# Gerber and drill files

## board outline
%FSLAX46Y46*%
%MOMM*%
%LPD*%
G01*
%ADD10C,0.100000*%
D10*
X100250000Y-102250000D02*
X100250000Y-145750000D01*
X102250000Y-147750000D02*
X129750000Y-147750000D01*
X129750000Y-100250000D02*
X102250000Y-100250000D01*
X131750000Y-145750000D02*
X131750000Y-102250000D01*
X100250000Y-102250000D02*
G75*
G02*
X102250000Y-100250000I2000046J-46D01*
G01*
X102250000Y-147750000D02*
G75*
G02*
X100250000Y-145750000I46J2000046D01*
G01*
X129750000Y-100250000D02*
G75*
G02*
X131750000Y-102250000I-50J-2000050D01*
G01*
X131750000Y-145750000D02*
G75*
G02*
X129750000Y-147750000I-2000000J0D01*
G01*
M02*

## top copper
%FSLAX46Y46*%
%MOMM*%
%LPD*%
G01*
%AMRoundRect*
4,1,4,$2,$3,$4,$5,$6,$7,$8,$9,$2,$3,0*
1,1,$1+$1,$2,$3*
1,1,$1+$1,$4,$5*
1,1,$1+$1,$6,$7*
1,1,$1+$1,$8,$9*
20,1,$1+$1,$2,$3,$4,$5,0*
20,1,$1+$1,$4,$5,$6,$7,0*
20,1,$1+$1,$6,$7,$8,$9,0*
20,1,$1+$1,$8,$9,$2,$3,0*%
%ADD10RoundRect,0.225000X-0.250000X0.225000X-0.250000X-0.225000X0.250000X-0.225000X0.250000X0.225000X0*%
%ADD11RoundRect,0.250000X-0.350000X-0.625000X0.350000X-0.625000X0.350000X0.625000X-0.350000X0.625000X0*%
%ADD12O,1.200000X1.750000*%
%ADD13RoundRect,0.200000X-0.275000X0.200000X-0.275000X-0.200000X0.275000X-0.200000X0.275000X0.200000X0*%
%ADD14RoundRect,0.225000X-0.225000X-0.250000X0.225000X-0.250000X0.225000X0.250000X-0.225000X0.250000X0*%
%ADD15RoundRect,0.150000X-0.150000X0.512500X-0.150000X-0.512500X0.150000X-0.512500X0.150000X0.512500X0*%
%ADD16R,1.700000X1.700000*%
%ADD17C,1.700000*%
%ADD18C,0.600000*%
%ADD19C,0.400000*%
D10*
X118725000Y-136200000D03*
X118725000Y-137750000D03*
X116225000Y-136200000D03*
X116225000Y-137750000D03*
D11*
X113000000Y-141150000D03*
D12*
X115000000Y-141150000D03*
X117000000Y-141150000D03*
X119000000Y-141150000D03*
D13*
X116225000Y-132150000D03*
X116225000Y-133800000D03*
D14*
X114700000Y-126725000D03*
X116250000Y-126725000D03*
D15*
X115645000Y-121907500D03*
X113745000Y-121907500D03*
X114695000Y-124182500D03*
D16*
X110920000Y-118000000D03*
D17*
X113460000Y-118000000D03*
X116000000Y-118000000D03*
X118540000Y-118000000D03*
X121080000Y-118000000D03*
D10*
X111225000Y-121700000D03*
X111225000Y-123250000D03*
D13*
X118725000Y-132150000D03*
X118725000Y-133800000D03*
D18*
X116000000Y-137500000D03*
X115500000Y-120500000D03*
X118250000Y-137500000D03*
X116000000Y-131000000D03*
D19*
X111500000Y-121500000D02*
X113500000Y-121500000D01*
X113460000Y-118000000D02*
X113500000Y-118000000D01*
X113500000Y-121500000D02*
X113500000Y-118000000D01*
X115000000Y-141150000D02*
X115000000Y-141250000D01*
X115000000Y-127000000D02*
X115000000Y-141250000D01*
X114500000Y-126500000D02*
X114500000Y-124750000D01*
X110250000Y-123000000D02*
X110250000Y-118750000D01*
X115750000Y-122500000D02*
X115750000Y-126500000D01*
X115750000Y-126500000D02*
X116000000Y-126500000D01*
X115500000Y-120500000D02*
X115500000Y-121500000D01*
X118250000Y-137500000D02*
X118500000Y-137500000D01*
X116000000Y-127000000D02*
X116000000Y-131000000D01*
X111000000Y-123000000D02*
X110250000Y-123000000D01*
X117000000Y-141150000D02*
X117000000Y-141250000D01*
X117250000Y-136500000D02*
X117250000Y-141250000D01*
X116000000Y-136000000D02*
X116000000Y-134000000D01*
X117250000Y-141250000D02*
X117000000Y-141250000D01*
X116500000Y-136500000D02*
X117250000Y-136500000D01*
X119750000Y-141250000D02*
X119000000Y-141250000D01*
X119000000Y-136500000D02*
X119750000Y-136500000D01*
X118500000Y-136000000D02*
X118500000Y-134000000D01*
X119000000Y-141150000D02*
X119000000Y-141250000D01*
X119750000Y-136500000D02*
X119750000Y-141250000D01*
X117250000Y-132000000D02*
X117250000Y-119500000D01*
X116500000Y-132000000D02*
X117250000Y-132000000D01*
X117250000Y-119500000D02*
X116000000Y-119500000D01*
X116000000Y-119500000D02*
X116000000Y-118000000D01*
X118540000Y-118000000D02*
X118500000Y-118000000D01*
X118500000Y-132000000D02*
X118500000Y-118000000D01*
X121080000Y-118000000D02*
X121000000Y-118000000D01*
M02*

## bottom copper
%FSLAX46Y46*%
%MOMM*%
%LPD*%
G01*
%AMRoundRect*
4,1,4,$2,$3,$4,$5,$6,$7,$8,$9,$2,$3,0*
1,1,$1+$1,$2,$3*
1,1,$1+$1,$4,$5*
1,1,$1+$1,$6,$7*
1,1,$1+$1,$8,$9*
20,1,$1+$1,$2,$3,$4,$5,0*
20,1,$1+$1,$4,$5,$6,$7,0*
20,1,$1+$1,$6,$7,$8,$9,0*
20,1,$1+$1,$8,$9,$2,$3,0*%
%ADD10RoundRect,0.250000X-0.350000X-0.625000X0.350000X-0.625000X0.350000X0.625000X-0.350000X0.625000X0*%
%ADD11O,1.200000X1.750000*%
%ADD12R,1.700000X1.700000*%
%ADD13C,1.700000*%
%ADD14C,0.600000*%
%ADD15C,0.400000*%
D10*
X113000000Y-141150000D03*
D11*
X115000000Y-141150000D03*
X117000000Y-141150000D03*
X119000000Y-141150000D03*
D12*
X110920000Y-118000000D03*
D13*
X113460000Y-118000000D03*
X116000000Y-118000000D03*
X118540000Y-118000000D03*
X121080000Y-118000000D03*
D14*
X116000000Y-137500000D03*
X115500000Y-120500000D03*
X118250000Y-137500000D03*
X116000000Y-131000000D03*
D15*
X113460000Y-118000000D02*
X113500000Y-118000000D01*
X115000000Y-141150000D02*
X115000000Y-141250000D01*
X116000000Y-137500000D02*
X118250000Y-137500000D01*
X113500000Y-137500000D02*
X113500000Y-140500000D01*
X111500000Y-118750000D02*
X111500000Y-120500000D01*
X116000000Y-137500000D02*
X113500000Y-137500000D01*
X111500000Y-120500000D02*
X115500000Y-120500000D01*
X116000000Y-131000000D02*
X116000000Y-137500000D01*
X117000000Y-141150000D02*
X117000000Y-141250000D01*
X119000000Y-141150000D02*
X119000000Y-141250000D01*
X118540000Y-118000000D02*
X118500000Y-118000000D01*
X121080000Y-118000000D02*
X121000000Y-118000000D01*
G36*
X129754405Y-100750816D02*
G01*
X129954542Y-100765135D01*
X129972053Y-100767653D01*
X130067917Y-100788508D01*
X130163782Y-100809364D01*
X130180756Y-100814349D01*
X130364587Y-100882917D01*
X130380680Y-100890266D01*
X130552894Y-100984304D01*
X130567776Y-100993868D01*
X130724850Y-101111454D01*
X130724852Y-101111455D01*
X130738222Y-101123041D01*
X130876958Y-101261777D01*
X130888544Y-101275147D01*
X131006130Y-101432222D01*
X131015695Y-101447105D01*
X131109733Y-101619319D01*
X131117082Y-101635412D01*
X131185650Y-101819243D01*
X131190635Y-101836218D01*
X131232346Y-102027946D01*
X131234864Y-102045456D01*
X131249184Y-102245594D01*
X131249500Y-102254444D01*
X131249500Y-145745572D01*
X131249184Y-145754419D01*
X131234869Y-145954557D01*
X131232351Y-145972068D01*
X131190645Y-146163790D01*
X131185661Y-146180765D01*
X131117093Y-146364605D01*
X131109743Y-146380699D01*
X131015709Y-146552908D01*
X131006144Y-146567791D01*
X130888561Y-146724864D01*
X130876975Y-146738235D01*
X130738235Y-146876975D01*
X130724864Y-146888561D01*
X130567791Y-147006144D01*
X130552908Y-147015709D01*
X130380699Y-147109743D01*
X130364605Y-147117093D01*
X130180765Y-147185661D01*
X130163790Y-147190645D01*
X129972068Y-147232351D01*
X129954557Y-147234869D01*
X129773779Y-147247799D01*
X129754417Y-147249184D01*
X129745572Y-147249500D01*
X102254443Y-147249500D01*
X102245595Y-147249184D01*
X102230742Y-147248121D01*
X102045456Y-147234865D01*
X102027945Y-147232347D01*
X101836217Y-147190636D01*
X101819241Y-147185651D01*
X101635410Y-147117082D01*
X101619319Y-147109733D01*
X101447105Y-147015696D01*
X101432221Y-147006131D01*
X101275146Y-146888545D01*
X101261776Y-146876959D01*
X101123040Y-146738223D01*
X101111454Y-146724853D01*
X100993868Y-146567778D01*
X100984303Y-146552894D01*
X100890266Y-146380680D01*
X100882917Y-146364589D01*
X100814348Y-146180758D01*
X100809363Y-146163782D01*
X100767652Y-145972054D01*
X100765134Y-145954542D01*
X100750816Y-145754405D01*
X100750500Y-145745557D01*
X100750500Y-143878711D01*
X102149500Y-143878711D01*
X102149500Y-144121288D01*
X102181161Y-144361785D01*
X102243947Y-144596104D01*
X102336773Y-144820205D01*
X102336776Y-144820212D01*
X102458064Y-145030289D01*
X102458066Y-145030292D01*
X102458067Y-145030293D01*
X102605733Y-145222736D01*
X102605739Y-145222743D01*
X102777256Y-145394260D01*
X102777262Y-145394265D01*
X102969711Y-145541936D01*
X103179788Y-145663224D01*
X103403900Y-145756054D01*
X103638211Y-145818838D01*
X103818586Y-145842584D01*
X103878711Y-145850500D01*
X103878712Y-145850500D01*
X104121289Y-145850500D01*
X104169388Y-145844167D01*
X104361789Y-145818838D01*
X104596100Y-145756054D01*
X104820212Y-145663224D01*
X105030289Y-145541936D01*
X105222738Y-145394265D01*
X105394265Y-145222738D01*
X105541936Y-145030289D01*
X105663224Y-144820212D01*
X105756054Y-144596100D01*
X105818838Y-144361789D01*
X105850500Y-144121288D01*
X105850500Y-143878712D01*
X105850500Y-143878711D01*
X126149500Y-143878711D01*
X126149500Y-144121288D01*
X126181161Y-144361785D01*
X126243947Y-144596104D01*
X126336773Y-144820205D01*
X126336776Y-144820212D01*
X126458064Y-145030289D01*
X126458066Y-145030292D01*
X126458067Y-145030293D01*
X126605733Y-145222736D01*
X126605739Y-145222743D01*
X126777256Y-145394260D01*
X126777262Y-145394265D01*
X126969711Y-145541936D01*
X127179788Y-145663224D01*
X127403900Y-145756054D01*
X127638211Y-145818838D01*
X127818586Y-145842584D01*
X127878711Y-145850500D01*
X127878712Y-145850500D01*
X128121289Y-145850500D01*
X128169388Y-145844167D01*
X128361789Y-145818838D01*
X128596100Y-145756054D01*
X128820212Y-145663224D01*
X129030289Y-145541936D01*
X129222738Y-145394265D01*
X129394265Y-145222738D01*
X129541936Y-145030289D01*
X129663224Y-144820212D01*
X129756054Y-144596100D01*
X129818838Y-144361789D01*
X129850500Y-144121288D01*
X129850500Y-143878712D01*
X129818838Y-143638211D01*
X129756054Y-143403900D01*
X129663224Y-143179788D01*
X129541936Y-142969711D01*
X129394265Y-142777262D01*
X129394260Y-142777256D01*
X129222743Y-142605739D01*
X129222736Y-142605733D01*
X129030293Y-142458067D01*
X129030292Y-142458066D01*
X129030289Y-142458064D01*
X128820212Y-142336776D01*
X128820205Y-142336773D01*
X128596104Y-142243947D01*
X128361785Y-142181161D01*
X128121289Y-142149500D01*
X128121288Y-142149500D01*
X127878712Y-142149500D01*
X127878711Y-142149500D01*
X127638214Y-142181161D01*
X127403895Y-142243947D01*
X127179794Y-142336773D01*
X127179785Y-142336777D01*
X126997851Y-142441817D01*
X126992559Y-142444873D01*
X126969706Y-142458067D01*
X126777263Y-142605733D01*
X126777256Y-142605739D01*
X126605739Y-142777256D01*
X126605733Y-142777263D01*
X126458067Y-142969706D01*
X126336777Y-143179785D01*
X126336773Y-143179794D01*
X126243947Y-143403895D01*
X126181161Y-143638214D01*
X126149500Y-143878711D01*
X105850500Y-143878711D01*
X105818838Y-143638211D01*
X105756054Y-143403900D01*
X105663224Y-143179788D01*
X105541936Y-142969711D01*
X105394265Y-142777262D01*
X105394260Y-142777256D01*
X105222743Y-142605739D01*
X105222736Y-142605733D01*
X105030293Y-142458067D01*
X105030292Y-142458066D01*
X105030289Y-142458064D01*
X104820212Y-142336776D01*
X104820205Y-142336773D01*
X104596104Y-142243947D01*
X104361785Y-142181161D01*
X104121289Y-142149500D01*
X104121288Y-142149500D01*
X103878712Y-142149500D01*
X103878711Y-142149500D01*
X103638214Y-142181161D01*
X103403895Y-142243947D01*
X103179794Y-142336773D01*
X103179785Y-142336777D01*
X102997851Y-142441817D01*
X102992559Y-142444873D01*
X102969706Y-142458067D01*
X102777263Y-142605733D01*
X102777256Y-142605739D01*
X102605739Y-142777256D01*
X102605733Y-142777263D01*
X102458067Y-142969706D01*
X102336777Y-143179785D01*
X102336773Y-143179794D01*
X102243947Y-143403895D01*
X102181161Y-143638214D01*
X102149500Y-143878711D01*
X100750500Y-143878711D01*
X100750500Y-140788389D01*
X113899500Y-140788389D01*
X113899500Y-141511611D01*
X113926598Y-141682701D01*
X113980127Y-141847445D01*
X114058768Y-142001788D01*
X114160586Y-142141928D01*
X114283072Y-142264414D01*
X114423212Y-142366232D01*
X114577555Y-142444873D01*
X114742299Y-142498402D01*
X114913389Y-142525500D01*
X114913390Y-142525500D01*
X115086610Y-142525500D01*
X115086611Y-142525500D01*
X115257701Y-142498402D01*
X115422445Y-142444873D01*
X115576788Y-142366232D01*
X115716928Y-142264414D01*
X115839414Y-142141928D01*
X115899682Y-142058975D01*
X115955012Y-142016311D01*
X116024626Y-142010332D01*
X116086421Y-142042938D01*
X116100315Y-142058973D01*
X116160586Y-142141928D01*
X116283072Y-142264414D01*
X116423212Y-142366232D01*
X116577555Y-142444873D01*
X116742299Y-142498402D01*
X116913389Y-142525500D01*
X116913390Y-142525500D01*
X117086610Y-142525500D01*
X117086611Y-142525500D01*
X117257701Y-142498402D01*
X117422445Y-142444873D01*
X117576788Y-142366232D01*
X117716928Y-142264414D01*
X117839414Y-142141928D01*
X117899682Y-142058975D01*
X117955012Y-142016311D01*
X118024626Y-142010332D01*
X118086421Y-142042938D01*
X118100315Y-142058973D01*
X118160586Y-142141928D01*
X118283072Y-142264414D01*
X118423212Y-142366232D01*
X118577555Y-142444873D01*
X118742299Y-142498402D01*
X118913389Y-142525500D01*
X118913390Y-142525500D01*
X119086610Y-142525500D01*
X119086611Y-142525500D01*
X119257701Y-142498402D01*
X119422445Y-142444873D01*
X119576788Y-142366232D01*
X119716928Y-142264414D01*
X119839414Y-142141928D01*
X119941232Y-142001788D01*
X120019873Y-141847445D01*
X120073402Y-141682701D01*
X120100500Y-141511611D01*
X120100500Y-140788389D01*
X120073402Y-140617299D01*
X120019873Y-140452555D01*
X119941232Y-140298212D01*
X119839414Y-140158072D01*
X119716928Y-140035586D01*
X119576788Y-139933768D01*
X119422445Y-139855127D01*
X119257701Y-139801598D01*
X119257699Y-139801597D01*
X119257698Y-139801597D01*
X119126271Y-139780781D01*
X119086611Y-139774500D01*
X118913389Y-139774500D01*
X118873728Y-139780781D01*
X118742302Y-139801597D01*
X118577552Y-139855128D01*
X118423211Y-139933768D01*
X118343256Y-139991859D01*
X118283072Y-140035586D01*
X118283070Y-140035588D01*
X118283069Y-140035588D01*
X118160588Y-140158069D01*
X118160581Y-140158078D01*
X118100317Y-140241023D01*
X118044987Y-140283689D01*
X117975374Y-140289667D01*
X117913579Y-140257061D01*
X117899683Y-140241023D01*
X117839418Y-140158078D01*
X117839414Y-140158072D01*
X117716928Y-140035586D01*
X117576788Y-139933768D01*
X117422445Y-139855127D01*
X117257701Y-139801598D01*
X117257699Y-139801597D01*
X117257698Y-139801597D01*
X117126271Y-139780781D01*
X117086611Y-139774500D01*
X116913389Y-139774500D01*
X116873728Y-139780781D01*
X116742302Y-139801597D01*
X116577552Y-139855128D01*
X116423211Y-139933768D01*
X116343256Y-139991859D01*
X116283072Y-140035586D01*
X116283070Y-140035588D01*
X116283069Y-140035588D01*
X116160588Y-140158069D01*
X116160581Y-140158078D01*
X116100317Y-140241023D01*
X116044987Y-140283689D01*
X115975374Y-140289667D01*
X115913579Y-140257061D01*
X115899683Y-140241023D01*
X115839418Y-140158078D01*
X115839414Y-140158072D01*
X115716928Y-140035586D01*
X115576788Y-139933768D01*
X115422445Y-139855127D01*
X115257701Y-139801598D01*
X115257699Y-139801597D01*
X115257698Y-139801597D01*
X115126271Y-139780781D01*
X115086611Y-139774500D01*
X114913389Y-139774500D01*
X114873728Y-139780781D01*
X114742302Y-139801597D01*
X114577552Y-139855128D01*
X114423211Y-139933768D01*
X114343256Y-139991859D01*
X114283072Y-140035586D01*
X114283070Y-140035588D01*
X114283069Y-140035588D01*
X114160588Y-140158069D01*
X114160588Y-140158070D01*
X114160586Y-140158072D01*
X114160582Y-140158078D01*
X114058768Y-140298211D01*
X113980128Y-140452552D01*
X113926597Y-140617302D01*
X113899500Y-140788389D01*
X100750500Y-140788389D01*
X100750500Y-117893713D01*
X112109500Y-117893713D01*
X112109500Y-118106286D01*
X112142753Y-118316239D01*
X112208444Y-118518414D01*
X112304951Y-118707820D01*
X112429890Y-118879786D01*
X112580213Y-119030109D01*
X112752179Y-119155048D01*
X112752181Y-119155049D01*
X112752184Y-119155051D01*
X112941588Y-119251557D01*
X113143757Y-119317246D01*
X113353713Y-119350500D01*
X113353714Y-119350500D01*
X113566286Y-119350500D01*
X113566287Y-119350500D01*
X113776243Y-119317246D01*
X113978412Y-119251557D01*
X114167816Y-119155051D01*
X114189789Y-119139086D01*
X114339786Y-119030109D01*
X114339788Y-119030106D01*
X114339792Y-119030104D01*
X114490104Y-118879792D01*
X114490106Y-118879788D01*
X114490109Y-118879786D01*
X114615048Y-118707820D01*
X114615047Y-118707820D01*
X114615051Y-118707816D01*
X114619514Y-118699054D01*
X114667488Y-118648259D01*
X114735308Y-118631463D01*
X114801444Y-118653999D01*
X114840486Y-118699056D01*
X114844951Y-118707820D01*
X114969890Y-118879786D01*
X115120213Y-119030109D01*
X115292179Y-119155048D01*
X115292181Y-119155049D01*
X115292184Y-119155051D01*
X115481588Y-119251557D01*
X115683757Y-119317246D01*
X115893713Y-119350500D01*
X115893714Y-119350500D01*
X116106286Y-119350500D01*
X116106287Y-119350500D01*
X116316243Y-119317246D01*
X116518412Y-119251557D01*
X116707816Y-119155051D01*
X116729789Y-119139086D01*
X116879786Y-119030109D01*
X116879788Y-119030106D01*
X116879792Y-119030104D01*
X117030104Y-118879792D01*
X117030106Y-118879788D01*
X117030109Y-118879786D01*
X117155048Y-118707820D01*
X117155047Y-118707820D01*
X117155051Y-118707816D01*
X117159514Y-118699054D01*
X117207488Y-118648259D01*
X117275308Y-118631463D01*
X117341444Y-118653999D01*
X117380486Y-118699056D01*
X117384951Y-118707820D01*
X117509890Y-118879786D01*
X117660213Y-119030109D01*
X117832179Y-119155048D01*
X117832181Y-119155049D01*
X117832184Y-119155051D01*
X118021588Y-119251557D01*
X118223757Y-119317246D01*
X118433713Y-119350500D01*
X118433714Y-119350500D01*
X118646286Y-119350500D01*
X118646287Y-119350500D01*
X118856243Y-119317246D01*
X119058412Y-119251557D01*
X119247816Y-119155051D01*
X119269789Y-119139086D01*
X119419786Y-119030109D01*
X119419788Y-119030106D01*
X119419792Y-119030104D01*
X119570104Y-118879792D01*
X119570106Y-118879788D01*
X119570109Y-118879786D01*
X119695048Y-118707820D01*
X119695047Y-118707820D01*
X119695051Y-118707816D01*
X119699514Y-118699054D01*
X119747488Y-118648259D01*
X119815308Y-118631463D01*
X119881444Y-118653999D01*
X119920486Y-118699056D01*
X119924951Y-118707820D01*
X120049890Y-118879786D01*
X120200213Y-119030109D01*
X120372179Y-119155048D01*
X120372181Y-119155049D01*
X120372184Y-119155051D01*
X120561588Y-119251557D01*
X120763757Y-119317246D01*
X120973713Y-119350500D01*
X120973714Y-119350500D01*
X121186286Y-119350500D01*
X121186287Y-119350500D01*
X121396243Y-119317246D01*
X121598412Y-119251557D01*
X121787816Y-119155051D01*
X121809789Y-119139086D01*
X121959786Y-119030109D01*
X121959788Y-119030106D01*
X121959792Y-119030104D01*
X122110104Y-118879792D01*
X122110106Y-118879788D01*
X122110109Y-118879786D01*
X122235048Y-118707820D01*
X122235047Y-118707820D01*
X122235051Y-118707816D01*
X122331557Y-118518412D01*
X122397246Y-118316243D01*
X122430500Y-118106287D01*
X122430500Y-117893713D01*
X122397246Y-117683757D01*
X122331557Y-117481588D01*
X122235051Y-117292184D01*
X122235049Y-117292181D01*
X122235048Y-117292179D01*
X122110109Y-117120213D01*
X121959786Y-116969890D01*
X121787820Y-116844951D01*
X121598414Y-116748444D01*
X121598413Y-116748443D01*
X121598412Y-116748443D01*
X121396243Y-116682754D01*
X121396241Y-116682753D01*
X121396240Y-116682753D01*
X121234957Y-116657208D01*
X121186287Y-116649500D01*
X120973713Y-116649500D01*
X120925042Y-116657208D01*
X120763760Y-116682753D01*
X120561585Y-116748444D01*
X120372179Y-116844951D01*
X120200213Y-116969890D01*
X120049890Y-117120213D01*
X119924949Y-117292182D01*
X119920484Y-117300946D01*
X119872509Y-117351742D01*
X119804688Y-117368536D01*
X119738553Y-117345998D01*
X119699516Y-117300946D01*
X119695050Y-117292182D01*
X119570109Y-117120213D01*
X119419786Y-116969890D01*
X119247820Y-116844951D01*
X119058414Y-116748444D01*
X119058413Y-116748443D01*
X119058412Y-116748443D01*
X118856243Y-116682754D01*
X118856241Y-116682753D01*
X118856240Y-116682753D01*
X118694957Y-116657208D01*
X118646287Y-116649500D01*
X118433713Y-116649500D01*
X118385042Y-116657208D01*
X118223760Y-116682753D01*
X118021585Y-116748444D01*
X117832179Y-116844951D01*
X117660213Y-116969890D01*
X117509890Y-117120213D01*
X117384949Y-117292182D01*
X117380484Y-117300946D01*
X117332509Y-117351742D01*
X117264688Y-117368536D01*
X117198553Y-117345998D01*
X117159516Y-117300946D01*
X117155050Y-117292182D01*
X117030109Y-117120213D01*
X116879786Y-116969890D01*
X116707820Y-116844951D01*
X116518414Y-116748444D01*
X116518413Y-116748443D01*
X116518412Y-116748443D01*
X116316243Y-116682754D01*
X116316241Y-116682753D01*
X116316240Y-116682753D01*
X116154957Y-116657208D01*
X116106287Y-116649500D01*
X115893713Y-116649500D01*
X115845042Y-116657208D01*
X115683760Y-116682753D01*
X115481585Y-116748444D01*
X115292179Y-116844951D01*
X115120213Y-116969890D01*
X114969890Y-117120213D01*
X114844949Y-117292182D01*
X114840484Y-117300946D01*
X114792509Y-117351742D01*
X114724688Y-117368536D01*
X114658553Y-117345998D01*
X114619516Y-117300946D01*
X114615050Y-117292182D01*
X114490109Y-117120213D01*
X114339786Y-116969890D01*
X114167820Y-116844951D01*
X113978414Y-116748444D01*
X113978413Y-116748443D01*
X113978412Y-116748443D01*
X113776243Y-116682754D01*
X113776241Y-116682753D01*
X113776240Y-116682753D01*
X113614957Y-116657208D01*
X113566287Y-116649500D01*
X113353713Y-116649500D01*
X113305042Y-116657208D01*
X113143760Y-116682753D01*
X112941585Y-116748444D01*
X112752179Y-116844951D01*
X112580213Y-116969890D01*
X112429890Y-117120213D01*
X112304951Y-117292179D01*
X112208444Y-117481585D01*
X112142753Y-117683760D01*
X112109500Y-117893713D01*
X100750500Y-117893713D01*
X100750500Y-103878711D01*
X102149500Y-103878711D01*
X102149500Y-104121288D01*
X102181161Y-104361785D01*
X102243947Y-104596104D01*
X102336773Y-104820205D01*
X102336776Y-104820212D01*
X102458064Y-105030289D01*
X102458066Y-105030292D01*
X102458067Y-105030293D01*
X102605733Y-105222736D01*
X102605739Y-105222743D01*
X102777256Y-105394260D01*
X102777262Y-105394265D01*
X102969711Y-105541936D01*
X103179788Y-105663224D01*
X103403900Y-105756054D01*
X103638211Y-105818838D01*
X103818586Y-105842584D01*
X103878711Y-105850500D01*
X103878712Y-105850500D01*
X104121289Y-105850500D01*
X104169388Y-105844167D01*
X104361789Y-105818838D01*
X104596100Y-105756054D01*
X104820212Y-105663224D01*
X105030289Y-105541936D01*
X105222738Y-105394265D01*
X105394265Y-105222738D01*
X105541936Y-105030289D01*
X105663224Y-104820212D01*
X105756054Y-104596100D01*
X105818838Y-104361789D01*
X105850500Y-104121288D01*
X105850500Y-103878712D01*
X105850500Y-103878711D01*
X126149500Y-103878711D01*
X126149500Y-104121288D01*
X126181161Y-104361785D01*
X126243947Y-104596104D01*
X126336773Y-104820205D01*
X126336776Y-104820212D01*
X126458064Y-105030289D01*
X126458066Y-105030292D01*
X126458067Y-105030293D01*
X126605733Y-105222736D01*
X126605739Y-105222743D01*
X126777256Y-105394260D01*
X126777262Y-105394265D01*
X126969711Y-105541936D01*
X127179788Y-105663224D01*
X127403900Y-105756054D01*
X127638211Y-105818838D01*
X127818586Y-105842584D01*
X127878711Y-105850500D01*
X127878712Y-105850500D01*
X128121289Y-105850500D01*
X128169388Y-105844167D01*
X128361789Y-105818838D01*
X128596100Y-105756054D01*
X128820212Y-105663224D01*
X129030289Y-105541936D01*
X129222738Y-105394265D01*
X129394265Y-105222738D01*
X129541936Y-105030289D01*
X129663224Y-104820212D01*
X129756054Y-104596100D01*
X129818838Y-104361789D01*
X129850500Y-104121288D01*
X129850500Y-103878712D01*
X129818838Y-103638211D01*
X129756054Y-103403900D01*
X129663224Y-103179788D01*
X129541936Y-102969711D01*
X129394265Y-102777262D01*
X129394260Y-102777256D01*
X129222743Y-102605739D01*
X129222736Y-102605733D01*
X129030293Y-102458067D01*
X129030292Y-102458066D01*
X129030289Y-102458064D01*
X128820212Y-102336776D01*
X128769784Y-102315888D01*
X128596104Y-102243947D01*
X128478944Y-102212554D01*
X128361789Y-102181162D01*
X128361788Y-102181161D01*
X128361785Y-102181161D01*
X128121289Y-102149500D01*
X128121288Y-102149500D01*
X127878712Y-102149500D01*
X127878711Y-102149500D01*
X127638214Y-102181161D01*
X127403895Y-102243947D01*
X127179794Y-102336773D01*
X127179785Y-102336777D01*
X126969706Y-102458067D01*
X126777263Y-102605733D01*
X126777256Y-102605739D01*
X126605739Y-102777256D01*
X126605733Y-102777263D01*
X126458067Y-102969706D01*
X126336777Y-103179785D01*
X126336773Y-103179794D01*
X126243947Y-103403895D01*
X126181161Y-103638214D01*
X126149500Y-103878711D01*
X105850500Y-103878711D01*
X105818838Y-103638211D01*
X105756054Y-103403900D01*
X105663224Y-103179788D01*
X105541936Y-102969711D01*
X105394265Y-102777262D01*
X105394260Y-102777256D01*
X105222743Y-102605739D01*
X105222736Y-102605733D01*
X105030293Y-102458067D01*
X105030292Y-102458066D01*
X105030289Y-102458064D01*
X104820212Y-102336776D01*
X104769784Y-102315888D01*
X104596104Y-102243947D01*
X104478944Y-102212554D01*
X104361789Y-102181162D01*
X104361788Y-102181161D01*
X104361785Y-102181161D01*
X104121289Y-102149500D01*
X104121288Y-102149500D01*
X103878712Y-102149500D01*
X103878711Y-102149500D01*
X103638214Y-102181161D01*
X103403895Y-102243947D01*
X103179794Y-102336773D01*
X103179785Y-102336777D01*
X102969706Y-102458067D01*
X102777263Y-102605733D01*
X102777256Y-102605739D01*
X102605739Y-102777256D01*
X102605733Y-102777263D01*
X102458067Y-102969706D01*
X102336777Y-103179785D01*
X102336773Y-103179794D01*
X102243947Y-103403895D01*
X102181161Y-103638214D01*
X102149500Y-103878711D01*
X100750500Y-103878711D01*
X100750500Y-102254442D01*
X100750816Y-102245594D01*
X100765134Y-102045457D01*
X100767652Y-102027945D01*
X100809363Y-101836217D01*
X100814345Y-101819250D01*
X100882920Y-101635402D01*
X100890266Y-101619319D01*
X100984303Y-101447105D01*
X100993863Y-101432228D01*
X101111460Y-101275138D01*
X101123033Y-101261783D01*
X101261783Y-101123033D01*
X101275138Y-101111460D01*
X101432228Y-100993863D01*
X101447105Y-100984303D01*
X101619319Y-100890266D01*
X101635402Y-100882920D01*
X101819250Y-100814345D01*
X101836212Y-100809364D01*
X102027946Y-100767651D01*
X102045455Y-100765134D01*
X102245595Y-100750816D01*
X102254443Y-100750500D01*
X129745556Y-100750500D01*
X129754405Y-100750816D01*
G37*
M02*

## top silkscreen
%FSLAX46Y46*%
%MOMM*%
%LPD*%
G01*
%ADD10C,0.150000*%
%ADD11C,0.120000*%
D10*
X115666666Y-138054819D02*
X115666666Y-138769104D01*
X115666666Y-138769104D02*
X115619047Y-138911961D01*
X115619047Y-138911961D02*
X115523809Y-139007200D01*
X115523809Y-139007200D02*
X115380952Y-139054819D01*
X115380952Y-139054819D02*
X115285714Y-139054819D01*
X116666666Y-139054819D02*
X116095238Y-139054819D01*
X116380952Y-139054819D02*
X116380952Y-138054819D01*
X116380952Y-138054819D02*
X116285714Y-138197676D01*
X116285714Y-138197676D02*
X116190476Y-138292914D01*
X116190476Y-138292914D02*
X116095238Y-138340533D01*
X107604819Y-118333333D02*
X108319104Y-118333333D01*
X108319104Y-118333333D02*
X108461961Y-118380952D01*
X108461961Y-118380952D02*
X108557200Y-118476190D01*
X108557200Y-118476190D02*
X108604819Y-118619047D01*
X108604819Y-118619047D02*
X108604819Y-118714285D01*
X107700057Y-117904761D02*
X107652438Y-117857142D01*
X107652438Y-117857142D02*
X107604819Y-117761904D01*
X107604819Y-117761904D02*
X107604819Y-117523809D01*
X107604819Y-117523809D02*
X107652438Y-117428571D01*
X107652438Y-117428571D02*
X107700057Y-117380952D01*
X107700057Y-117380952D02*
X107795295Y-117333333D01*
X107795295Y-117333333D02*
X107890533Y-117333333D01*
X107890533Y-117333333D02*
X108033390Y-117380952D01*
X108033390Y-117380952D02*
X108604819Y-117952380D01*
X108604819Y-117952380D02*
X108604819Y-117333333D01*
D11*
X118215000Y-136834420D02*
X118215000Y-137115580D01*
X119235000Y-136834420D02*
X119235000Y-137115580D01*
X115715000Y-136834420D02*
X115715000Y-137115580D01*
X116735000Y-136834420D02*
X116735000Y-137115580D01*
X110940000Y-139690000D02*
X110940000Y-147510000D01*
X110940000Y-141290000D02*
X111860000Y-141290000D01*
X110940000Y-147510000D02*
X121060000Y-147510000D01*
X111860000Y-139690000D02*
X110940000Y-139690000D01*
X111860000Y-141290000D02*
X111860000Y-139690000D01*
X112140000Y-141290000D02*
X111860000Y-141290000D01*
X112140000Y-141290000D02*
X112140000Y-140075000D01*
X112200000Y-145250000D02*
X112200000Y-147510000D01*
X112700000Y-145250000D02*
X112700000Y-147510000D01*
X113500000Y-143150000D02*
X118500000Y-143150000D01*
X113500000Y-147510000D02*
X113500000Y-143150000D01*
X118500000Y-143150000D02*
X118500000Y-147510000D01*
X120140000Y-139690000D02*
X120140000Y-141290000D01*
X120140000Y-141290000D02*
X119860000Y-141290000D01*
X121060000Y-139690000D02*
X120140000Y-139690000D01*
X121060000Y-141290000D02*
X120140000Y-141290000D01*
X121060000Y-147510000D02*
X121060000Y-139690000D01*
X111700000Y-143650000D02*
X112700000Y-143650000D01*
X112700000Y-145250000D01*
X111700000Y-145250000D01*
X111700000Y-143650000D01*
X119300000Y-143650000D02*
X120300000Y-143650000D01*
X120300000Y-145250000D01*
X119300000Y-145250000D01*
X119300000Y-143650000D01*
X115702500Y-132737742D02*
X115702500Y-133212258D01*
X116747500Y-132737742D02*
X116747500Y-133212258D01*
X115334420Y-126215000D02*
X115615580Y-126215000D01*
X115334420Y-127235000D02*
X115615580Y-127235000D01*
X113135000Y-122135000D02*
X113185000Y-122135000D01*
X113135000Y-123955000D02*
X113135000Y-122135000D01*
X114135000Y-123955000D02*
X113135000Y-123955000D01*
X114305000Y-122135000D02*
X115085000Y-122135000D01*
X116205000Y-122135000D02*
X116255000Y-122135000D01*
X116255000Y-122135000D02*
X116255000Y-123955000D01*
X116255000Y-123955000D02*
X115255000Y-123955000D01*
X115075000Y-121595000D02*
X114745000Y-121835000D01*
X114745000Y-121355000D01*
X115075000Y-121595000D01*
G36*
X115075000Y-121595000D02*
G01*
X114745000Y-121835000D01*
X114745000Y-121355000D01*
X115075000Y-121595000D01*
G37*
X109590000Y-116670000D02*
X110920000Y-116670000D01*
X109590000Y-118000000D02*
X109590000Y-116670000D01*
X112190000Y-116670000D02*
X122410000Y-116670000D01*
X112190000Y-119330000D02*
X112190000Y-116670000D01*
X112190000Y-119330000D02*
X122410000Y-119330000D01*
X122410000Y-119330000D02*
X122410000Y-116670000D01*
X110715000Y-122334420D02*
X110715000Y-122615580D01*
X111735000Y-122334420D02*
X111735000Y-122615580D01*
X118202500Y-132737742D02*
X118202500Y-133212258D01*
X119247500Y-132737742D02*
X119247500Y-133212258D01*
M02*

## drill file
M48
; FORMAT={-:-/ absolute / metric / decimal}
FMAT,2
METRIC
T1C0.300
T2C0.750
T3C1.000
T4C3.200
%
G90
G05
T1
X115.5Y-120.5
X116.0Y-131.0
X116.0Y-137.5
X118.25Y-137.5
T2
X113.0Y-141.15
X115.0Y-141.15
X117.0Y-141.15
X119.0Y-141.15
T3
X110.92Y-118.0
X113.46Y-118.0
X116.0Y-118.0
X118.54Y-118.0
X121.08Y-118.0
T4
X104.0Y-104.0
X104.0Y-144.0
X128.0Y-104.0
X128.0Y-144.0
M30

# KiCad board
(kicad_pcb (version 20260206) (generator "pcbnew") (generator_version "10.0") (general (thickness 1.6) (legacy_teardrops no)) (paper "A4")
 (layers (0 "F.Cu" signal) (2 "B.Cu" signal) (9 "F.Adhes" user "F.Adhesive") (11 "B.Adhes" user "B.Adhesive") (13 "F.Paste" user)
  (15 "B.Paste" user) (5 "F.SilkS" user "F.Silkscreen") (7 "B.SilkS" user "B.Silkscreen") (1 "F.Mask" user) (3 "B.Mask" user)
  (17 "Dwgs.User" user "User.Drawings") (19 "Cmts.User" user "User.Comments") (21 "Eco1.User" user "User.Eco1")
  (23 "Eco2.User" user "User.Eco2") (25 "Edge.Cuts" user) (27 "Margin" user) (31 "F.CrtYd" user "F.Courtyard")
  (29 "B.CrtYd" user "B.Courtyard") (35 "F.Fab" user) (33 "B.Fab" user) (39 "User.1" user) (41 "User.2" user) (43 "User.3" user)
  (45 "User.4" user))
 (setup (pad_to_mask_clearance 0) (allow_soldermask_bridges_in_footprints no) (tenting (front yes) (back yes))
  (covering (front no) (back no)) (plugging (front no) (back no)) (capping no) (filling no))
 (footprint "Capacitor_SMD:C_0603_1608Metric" (layer "F.Cu") (at 118.725 136.975 -90)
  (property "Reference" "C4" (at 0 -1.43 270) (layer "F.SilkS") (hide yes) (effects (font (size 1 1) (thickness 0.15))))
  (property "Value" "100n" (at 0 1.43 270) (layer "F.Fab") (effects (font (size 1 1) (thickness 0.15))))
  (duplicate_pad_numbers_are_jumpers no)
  (fp_line (start -0.14058 0.51) (end 0.14058 0.51) (stroke (width 0.12) (type solid)) (layer "F.SilkS"))
  (fp_line (start -0.14058 -0.51) (end 0.14058 -0.51) (stroke (width 0.12) (type solid)) (layer "F.SilkS"))
  (pad "1" smd roundrect (at -0.775 0 270) (size 0.9 0.95) (layers "F.Cu" "F.Mask" "F.Paste") (roundrect_rratio 0.25) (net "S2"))
  (pad "2" smd roundrect (at 0.775 0 270) (size 0.9 0.95) (layers "F.Cu" "F.Mask" "F.Paste") (roundrect_rratio 0.25) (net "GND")))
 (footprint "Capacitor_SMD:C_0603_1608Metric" (layer "F.Cu") (at 116.225 136.975 -90)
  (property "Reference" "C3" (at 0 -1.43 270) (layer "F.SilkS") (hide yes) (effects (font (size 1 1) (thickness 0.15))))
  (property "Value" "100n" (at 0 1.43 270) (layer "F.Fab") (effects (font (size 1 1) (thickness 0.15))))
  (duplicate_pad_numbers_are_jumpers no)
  (fp_line (start -0.14058 0.51) (end 0.14058 0.51) (stroke (width 0.12) (type solid)) (layer "F.SilkS"))
  (fp_line (start -0.14058 -0.51) (end 0.14058 -0.51) (stroke (width 0.12) (type solid)) (layer "F.SilkS"))
  (pad "1" smd roundrect (at -0.775 0 270) (size 0.9 0.95) (layers "F.Cu" "F.Mask" "F.Paste") (roundrect_rratio 0.25) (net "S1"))
  (pad "2" smd roundrect (at 0.775 0 270) (size 0.9 0.95) (layers "F.Cu" "F.Mask" "F.Paste") (roundrect_rratio 0.25) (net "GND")))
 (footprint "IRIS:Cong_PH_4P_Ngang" (layer "F.Cu") (at 113 141.15)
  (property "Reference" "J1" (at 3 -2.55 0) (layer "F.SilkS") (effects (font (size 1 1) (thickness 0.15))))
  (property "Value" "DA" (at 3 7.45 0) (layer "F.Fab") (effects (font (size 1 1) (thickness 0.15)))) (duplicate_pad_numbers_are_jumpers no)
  (fp_line (start -2.06 -1.46) (end -2.06 6.36) (stroke (width 0.12) (type solid)) (layer "F.SilkS"))
  (fp_line (start -2.06 0.14) (end -1.14 0.14) (stroke (width 0.12) (type solid)) (layer "F.SilkS"))
  (fp_line (start -2.06 6.36) (end 8.06 6.36) (stroke (width 0.12) (type solid)) (layer "F.SilkS"))
  (fp_line (start -1.14 -1.46) (end -2.06 -1.46) (stroke (width 0.12) (type solid)) (layer "F.SilkS"))
  (fp_line (start -1.14 0.14) (end -1.14 -1.46) (stroke (width 0.12) (type solid)) (layer "F.SilkS"))
  (fp_line (start -0.86 0.14) (end -1.14 0.14) (stroke (width 0.12) (type solid)) (layer "F.SilkS"))
  (fp_line (start -0.86 0.14) (end -0.86 -1.075) (stroke (width 0.12) (type solid)) (layer "F.SilkS"))
  (fp_line (start -0.8 4.1) (end -0.8 6.36) (stroke (width 0.12) (type solid)) (layer "F.SilkS"))
  (fp_line (start -0.3 4.1) (end -0.3 6.36) (stroke (width 0.12) (type solid)) (layer "F.SilkS"))
  (fp_line (start 0.5 2) (end 5.5 2) (stroke (width 0.12) (type solid)) (layer "F.SilkS"))
  (fp_line (start 0.5 6.36) (end 0.5 2) (stroke (width 0.12) (type solid)) (layer "F.SilkS"))
  (fp_line (start 5.5 2) (end 5.5 6.36) (stroke (width 0.12) (type solid)) (layer "F.SilkS"))
  (fp_line (start 7.14 -1.46) (end 7.14 0.14) (stroke (width 0.12) (type solid)) (layer "F.SilkS"))
  (fp_line (start 7.14 0.14) (end 6.86 0.14) (stroke (width 0.12) (type solid)) (layer "F.SilkS"))
  (fp_line (start 8.06 -1.46) (end 7.14 -1.46) (stroke (width 0.12) (type solid)) (layer "F.SilkS"))
  (fp_line (start 8.06 0.14) (end 7.14 0.14) (stroke (width 0.12) (type solid)) (layer "F.SilkS"))
  (fp_line (start 8.06 6.36) (end 8.06 -1.46) (stroke (width 0.12) (type solid)) (layer "F.SilkS"))
  (fp_rect (start -1.3 2.5) (end -0.3 4.1) (stroke (width 0.12) (type solid)) (fill no) (layer "F.SilkS"))
  (fp_rect (start 6.3 2.5) (end 7.3 4.1) (stroke (width 0.12) (type solid)) (fill no) (layer "F.SilkS"))
  (pad "1" thru_hole roundrect (at 0 0) (size 1.2 1.75) (drill 0.75) (layers "*.Cu" "*.Mask") (remove_unused_layers no)
   (roundrect_rratio 0.208333) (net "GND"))
  (pad "2" thru_hole oval (at 2 0) (size 1.2 1.75) (drill 0.75) (layers "*.Cu" "*.Mask") (remove_unused_layers no) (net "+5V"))
  (pad "3" thru_hole oval (at 4 0) (size 1.2 1.75) (drill 0.75) (layers "*.Cu" "*.Mask") (remove_unused_layers no) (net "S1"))
  (pad "4" thru_hole oval (at 6 0) (size 1.2 1.75) (drill 0.75) (layers "*.Cu" "*.Mask") (remove_unused_layers no) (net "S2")))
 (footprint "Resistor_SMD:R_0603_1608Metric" (layer "F.Cu") (at 116.225 132.975 -90)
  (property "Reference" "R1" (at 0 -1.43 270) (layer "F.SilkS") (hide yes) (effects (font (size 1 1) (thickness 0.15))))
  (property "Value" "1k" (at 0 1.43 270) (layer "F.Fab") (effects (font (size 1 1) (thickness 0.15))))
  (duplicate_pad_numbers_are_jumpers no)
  (fp_line (start -0.237258 0.5225) (end 0.237258 0.5225) (stroke (width 0.12) (type solid)) (layer "F.SilkS"))
  (fp_line (start -0.237258 -0.5225) (end 0.237258 -0.5225) (stroke (width 0.12) (type solid)) (layer "F.SilkS"))
  (pad "1" smd roundrect (at -0.825 0 270) (size 0.8 0.95) (layers "F.Cu" "F.Mask" "F.Paste") (roundrect_rratio 0.25) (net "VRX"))
  (pad "2" smd roundrect (at 0.825 0 270) (size 0.8 0.95) (layers "F.Cu" "F.Mask" "F.Paste") (roundrect_rratio 0.25) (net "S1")))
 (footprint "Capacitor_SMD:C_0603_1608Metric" (layer "F.Cu") (at 115.475 126.725)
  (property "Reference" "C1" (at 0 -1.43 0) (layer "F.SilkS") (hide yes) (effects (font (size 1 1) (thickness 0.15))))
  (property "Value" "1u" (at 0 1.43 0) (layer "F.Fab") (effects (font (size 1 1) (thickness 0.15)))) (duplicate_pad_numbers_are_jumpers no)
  (fp_line (start -0.14058 -0.51) (end 0.14058 -0.51) (stroke (width 0.12) (type solid)) (layer "F.SilkS"))
  (fp_line (start -0.14058 0.51) (end 0.14058 0.51) (stroke (width 0.12) (type solid)) (layer "F.SilkS"))
  (pad "1" smd roundrect (at -0.775 0) (size 0.9 0.95) (layers "F.Cu" "F.Mask" "F.Paste") (roundrect_rratio 0.25) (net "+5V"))
  (pad "2" smd roundrect (at 0.775 0) (size 0.9 0.95) (layers "F.Cu" "F.Mask" "F.Paste") (roundrect_rratio 0.25) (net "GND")))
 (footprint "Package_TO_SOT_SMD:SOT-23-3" (layer "F.Cu") (at 114.695 123.045 -90)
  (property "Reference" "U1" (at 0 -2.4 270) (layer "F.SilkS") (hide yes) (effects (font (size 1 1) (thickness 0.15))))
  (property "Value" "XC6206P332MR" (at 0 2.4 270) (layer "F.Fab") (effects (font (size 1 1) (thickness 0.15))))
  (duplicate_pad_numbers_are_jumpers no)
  (fp_line (start -0.91 1.56) (end -0.91 1.51) (stroke (width 0.12) (type solid)) (layer "F.SilkS"))
  (fp_line (start 0.91 1.56) (end -0.91 1.56) (stroke (width 0.12) (type solid)) (layer "F.SilkS"))
  (fp_line (start 0.91 0.56) (end 0.91 1.56) (stroke (width 0.12) (type solid)) (layer "F.SilkS"))
  (fp_line (start -0.91 0.39) (end -0.91 -0.39) (stroke (width 0.12) (type solid)) (layer "F.SilkS"))
  (fp_line (start -0.91 -1.51) (end -0.91 -1.56) (stroke (width 0.12) (type solid)) (layer "F.SilkS"))
  (fp_line (start -0.91 -1.56) (end 0.91 -1.56) (stroke (width 0.12) (type solid)) (layer "F.SilkS"))
  (fp_line (start 0.91 -1.56) (end 0.91 -0.56) (stroke (width 0.12) (type solid)) (layer "F.SilkS"))
  (fp_poly (pts (xy -1.45 -0.38) (xy -1.21 -0.05) (xy -1.69 -0.05)) (stroke (width 0.12) (type solid)) (fill yes) (layer "F.SilkS"))
  (pad "1" smd roundrect (at -1.1375 -0.95 270) (size 1.325 0.6) (layers "F.Cu" "F.Mask" "F.Paste") (roundrect_rratio 0.25) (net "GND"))
  (pad "2" smd roundrect (at -1.1375 0.95 270) (size 1.325 0.6) (layers "F.Cu" "F.Mask" "F.Paste") (roundrect_rratio 0.25) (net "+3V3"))
  (pad "3" smd roundrect (at 1.1375 0 270) (size 1.325 0.6) (layers "F.Cu" "F.Mask" "F.Paste") (roundrect_rratio 0.25) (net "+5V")))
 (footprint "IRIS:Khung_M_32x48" (layer "F.Cu") (at 100 148)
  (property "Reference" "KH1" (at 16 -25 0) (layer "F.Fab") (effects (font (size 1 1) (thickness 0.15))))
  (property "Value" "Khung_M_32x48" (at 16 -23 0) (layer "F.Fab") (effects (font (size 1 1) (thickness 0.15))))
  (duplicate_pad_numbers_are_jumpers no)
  (fp_line (start 0.25 -45.75) (end 0.25 -2.25) (stroke (width 0.1) (type solid)) (layer "Edge.Cuts"))
  (fp_line (start 2.25 -0.25) (end 29.75 -0.25) (stroke (width 0.1) (type solid)) (layer "Edge.Cuts"))
  (fp_line (start 29.75 -47.75) (end 2.25 -47.75) (stroke (width 0.1) (type solid)) (layer "Edge.Cuts"))
  (fp_line (start 31.75 -2.25) (end 31.75 -45.75) (stroke (width 0.1) (type solid)) (layer "Edge.Cuts"))
  (fp_arc (start 0.25 -45.75) (mid 0.8358 -47.1642) (end 2.25 -47.75) (stroke (width 0.1) (type solid)) (layer "Edge.Cuts"))
  (fp_arc (start 2.25 -0.25) (mid 0.8358 -0.8358) (end 0.25 -2.25) (stroke (width 0.1) (type solid)) (layer "Edge.Cuts"))
  (fp_arc (start 29.75 -47.75) (mid 31.164199 -47.164199) (end 31.75 -45.75) (stroke (width 0.1) (type solid)) (layer "Edge.Cuts"))
  (fp_arc (start 31.75 -2.25) (mid 31.164214 -0.835786) (end 29.75 -0.25) (stroke (width 0.1) (type solid)) (layer "Edge.Cuts"))
  (pad "" np_thru_hole circle (at 4 -44) (size 3.2 3.2) (drill 3.2) (layers "*.Cu" "*.Mask"))
  (pad "" np_thru_hole circle (at 4 -4) (size 3.2 3.2) (drill 3.2) (layers "*.Cu" "*.Mask"))
  (pad "" np_thru_hole circle (at 28 -44) (size 3.2 3.2) (drill 3.2) (layers "*.Cu" "*.Mask"))
  (pad "" np_thru_hole circle (at 28 -4) (size 3.2 3.2) (drill 3.2) (layers "*.Cu" "*.Mask")))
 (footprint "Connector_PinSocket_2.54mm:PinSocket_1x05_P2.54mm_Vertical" (layer "F.Cu") (at 110.92 118 90)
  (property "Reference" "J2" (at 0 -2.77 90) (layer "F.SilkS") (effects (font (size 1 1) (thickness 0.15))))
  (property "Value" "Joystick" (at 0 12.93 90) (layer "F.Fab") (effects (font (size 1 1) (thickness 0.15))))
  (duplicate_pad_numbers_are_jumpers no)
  (fp_line (start 1.33 -1.33) (end 1.33 0) (stroke (width 0.12) (type solid)) (layer "F.SilkS"))
  (fp_line (start 0 -1.33) (end 1.33 -1.33) (stroke (width 0.12) (type solid)) (layer "F.SilkS"))
  (fp_line (start 1.33 1.27) (end 1.33 11.49) (stroke (width 0.12) (type solid)) (layer "F.SilkS"))
  (fp_line (start -1.33 1.27) (end 1.33 1.27) (stroke (width 0.12) (type solid)) (layer "F.SilkS"))
  (fp_line (start -1.33 1.27) (end -1.33 11.49) (stroke (width 0.12) (type solid)) (layer "F.SilkS"))
  (fp_line (start -1.33 11.49) (end 1.33 11.49) (stroke (width 0.12) (type solid)) (layer "F.SilkS"))
  (pad "1" thru_hole rect (at 0 0 90) (size 1.7 1.7) (drill 1) (layers "*.Cu" "*.Mask") (remove_unused_layers no) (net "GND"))
  (pad "2" thru_hole circle (at 0 2.54 90) (size 1.7 1.7) (drill 1) (layers "*.Cu" "*.Mask") (remove_unused_layers no) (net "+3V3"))
  (pad "3" thru_hole circle (at 0 5.08 90) (size 1.7 1.7) (drill 1) (layers "*.Cu" "*.Mask") (remove_unused_layers no) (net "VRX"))
  (pad "4" thru_hole circle (at 0 7.62 90) (size 1.7 1.7) (drill 1) (layers "*.Cu" "*.Mask") (remove_unused_layers no) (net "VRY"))
  (pad "5" thru_hole circle (at 0 10.16 90) (size 1.7 1.7) (drill 1) (layers "*.Cu" "*.Mask") (remove_unused_layers no)
   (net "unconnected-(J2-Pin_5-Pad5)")))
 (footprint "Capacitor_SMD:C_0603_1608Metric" (layer "F.Cu") (at 111.225 122.475 -90)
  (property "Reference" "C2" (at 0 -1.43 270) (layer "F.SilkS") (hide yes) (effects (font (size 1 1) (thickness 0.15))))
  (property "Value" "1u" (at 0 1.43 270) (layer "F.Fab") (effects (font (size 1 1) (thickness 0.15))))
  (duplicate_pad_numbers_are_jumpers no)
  (fp_line (start -0.14058 0.51) (end 0.14058 0.51) (stroke (width 0.12) (type solid)) (layer "F.SilkS"))
  (fp_line (start -0.14058 -0.51) (end 0.14058 -0.51) (stroke (width 0.12) (type solid)) (layer "F.SilkS"))
  (pad "1" smd roundrect (at -0.775 0 270) (size 0.9 0.95) (layers "F.Cu" "F.Mask" "F.Paste") (roundrect_rratio 0.25) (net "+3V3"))
  (pad "2" smd roundrect (at 0.775 0 270) (size 0.9 0.95) (layers "F.Cu" "F.Mask" "F.Paste") (roundrect_rratio 0.25) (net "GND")))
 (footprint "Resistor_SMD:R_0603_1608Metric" (layer "F.Cu") (at 118.725 132.975 -90)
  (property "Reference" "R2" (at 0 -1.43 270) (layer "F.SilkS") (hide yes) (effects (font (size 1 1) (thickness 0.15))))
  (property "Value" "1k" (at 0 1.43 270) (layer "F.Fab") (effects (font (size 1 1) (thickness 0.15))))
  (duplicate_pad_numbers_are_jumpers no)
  (fp_line (start -0.237258 0.5225) (end 0.237258 0.5225) (stroke (width 0.12) (type solid)) (layer "F.SilkS"))
  (fp_line (start -0.237258 -0.5225) (end 0.237258 -0.5225) (stroke (width 0.12) (type solid)) (layer "F.SilkS"))
  (pad "1" smd roundrect (at -0.825 0 270) (size 0.8 0.95) (layers "F.Cu" "F.Mask" "F.Paste") (roundrect_rratio 0.25) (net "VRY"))
  (pad "2" smd roundrect (at 0.825 0 270) (size 0.8 0.95) (layers "F.Cu" "F.Mask" "F.Paste") (roundrect_rratio 0.25) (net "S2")))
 (segment (start 111.5 121.5) (end 113.5 121.5) (width 0.4) (layer "F.Cu") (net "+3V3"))
 (segment (start 113.46 118) (end 113.5 118) (width 0.4) (layer "F.Cu") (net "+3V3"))
 (segment (start 113.5 121.5) (end 113.5 118) (width 0.4) (layer "F.Cu") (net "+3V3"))
 (segment (start 113.46 118) (end 113.5 118) (width 0.4) (layer "B.Cu") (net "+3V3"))
 (segment (start 115 141.15) (end 115 141.25) (width 0.4) (layer "F.Cu") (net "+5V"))
 (segment (start 115 127) (end 115 141.25) (width 0.4) (layer "F.Cu") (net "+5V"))
 (segment (start 114.5 126.5) (end 114.5 124.75) (width 0.4) (layer "F.Cu") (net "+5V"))
 (segment (start 115 141.15) (end 115 141.25) (width 0.4) (layer "B.Cu") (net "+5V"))
 (segment (start 110.25 123) (end 110.25 118.75) (width 0.4) (layer "F.Cu") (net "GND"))
 (segment (start 115.75 122.5) (end 115.75 126.5) (width 0.4) (layer "F.Cu") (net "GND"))
 (segment (start 115.75 126.5) (end 116 126.5) (width 0.4) (layer "F.Cu") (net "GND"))
 (segment (start 115.5 120.5) (end 115.5 121.5) (width 0.4) (layer "F.Cu") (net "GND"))
 (segment (start 118.25 137.5) (end 118.5 137.5) (width 0.4) (layer "F.Cu") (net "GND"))
 (segment (start 116 127) (end 116 131) (width 0.4) (layer "F.Cu") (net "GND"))
 (segment (start 111 123) (end 110.25 123) (width 0.4) (layer "F.Cu") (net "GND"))
 (via (at 116 137.5) (size 0.6) (drill 0.3) (layers "F.Cu" "B.Cu") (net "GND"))
 (via (at 115.5 120.5) (size 0.6) (drill 0.3) (layers "F.Cu" "B.Cu") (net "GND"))
 (via (at 118.25 137.5) (size 0.6) (drill 0.3) (layers "F.Cu" "B.Cu") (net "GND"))
 (via (at 116 131) (size 0.6) (drill 0.3) (layers "F.Cu" "B.Cu") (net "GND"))
 (segment (start 116 137.5) (end 118.25 137.5) (width 0.4) (layer "B.Cu") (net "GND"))
 (segment (start 113.5 137.5) (end 113.5 140.5) (width 0.4) (layer "B.Cu") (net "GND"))
 (segment (start 111.5 118.75) (end 111.5 120.5) (width 0.4) (layer "B.Cu") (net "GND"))
 (segment (start 116 137.5) (end 113.5 137.5) (width 0.4) (layer "B.Cu") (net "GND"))
 (segment (start 111.5 120.5) (end 115.5 120.5) (width 0.4) (layer "B.Cu") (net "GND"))
 (segment (start 116 131) (end 116 137.5) (width 0.4) (layer "B.Cu") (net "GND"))
 (segment (start 117 141.15) (end 117 141.25) (width 0.4) (layer "F.Cu") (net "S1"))
 (segment (start 117.25 136.5) (end 117.25 141.25) (width 0.4) (layer "F.Cu") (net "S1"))
 (segment (start 116 136) (end 116 134) (width 0.4) (layer "F.Cu") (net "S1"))
 (segment (start 117.25 141.25) (end 117 141.25) (width 0.4) (layer "F.Cu") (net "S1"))
 (segment (start 116.5 136.5) (end 117.25 136.5) (width 0.4) (layer "F.Cu") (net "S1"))
 (segment (start 117 141.15) (end 117 141.25) (width 0.4) (layer "B.Cu") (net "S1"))
 (segment (start 119.75 141.25) (end 119 141.25) (width 0.4) (layer "F.Cu") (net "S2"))
 (segment (start 119 136.5) (end 119.75 136.5) (width 0.4) (layer "F.Cu") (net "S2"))
 (segment (start 118.5 136) (end 118.5 134) (width 0.4) (layer "F.Cu") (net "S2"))
 (segment (start 119 141.15) (end 119 141.25) (width 0.4) (layer "F.Cu") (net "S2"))
 (segment (start 119.75 136.5) (end 119.75 141.25) (width 0.4) (layer "F.Cu") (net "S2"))
 (segment (start 119 141.15) (end 119 141.25) (width 0.4) (layer "B.Cu") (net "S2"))
 (segment (start 117.25 132) (end 117.25 119.5) (width 0.4) (layer "F.Cu") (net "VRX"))
 (segment (start 116.5 132) (end 117.25 132) (width 0.4) (layer "F.Cu") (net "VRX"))
 (segment (start 117.25 119.5) (end 116 119.5) (width 0.4) (layer "F.Cu") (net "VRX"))
 (segment (start 116 119.5) (end 116 118) (width 0.4) (layer "F.Cu") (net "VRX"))
 (segment (start 118.54 118) (end 118.5 118) (width 0.4) (layer "F.Cu") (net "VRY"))
 (segment (start 118.5 132) (end 118.5 118) (width 0.4) (layer "F.Cu") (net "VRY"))
 (segment (start 118.54 118) (end 118.5 118) (width 0.4) (layer "B.Cu") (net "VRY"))
 (segment (start 121.08 118) (end 121 118) (width 0.4) (layer "F.Cu") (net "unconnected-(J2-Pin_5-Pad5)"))
 (segment (start 121.08 118) (end 121 118) (width 0.4) (layer "B.Cu") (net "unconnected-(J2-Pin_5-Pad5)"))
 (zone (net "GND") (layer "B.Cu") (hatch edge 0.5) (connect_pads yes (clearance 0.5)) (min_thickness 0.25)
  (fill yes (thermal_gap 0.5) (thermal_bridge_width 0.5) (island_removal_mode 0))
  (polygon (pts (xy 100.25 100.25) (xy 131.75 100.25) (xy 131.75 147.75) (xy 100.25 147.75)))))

